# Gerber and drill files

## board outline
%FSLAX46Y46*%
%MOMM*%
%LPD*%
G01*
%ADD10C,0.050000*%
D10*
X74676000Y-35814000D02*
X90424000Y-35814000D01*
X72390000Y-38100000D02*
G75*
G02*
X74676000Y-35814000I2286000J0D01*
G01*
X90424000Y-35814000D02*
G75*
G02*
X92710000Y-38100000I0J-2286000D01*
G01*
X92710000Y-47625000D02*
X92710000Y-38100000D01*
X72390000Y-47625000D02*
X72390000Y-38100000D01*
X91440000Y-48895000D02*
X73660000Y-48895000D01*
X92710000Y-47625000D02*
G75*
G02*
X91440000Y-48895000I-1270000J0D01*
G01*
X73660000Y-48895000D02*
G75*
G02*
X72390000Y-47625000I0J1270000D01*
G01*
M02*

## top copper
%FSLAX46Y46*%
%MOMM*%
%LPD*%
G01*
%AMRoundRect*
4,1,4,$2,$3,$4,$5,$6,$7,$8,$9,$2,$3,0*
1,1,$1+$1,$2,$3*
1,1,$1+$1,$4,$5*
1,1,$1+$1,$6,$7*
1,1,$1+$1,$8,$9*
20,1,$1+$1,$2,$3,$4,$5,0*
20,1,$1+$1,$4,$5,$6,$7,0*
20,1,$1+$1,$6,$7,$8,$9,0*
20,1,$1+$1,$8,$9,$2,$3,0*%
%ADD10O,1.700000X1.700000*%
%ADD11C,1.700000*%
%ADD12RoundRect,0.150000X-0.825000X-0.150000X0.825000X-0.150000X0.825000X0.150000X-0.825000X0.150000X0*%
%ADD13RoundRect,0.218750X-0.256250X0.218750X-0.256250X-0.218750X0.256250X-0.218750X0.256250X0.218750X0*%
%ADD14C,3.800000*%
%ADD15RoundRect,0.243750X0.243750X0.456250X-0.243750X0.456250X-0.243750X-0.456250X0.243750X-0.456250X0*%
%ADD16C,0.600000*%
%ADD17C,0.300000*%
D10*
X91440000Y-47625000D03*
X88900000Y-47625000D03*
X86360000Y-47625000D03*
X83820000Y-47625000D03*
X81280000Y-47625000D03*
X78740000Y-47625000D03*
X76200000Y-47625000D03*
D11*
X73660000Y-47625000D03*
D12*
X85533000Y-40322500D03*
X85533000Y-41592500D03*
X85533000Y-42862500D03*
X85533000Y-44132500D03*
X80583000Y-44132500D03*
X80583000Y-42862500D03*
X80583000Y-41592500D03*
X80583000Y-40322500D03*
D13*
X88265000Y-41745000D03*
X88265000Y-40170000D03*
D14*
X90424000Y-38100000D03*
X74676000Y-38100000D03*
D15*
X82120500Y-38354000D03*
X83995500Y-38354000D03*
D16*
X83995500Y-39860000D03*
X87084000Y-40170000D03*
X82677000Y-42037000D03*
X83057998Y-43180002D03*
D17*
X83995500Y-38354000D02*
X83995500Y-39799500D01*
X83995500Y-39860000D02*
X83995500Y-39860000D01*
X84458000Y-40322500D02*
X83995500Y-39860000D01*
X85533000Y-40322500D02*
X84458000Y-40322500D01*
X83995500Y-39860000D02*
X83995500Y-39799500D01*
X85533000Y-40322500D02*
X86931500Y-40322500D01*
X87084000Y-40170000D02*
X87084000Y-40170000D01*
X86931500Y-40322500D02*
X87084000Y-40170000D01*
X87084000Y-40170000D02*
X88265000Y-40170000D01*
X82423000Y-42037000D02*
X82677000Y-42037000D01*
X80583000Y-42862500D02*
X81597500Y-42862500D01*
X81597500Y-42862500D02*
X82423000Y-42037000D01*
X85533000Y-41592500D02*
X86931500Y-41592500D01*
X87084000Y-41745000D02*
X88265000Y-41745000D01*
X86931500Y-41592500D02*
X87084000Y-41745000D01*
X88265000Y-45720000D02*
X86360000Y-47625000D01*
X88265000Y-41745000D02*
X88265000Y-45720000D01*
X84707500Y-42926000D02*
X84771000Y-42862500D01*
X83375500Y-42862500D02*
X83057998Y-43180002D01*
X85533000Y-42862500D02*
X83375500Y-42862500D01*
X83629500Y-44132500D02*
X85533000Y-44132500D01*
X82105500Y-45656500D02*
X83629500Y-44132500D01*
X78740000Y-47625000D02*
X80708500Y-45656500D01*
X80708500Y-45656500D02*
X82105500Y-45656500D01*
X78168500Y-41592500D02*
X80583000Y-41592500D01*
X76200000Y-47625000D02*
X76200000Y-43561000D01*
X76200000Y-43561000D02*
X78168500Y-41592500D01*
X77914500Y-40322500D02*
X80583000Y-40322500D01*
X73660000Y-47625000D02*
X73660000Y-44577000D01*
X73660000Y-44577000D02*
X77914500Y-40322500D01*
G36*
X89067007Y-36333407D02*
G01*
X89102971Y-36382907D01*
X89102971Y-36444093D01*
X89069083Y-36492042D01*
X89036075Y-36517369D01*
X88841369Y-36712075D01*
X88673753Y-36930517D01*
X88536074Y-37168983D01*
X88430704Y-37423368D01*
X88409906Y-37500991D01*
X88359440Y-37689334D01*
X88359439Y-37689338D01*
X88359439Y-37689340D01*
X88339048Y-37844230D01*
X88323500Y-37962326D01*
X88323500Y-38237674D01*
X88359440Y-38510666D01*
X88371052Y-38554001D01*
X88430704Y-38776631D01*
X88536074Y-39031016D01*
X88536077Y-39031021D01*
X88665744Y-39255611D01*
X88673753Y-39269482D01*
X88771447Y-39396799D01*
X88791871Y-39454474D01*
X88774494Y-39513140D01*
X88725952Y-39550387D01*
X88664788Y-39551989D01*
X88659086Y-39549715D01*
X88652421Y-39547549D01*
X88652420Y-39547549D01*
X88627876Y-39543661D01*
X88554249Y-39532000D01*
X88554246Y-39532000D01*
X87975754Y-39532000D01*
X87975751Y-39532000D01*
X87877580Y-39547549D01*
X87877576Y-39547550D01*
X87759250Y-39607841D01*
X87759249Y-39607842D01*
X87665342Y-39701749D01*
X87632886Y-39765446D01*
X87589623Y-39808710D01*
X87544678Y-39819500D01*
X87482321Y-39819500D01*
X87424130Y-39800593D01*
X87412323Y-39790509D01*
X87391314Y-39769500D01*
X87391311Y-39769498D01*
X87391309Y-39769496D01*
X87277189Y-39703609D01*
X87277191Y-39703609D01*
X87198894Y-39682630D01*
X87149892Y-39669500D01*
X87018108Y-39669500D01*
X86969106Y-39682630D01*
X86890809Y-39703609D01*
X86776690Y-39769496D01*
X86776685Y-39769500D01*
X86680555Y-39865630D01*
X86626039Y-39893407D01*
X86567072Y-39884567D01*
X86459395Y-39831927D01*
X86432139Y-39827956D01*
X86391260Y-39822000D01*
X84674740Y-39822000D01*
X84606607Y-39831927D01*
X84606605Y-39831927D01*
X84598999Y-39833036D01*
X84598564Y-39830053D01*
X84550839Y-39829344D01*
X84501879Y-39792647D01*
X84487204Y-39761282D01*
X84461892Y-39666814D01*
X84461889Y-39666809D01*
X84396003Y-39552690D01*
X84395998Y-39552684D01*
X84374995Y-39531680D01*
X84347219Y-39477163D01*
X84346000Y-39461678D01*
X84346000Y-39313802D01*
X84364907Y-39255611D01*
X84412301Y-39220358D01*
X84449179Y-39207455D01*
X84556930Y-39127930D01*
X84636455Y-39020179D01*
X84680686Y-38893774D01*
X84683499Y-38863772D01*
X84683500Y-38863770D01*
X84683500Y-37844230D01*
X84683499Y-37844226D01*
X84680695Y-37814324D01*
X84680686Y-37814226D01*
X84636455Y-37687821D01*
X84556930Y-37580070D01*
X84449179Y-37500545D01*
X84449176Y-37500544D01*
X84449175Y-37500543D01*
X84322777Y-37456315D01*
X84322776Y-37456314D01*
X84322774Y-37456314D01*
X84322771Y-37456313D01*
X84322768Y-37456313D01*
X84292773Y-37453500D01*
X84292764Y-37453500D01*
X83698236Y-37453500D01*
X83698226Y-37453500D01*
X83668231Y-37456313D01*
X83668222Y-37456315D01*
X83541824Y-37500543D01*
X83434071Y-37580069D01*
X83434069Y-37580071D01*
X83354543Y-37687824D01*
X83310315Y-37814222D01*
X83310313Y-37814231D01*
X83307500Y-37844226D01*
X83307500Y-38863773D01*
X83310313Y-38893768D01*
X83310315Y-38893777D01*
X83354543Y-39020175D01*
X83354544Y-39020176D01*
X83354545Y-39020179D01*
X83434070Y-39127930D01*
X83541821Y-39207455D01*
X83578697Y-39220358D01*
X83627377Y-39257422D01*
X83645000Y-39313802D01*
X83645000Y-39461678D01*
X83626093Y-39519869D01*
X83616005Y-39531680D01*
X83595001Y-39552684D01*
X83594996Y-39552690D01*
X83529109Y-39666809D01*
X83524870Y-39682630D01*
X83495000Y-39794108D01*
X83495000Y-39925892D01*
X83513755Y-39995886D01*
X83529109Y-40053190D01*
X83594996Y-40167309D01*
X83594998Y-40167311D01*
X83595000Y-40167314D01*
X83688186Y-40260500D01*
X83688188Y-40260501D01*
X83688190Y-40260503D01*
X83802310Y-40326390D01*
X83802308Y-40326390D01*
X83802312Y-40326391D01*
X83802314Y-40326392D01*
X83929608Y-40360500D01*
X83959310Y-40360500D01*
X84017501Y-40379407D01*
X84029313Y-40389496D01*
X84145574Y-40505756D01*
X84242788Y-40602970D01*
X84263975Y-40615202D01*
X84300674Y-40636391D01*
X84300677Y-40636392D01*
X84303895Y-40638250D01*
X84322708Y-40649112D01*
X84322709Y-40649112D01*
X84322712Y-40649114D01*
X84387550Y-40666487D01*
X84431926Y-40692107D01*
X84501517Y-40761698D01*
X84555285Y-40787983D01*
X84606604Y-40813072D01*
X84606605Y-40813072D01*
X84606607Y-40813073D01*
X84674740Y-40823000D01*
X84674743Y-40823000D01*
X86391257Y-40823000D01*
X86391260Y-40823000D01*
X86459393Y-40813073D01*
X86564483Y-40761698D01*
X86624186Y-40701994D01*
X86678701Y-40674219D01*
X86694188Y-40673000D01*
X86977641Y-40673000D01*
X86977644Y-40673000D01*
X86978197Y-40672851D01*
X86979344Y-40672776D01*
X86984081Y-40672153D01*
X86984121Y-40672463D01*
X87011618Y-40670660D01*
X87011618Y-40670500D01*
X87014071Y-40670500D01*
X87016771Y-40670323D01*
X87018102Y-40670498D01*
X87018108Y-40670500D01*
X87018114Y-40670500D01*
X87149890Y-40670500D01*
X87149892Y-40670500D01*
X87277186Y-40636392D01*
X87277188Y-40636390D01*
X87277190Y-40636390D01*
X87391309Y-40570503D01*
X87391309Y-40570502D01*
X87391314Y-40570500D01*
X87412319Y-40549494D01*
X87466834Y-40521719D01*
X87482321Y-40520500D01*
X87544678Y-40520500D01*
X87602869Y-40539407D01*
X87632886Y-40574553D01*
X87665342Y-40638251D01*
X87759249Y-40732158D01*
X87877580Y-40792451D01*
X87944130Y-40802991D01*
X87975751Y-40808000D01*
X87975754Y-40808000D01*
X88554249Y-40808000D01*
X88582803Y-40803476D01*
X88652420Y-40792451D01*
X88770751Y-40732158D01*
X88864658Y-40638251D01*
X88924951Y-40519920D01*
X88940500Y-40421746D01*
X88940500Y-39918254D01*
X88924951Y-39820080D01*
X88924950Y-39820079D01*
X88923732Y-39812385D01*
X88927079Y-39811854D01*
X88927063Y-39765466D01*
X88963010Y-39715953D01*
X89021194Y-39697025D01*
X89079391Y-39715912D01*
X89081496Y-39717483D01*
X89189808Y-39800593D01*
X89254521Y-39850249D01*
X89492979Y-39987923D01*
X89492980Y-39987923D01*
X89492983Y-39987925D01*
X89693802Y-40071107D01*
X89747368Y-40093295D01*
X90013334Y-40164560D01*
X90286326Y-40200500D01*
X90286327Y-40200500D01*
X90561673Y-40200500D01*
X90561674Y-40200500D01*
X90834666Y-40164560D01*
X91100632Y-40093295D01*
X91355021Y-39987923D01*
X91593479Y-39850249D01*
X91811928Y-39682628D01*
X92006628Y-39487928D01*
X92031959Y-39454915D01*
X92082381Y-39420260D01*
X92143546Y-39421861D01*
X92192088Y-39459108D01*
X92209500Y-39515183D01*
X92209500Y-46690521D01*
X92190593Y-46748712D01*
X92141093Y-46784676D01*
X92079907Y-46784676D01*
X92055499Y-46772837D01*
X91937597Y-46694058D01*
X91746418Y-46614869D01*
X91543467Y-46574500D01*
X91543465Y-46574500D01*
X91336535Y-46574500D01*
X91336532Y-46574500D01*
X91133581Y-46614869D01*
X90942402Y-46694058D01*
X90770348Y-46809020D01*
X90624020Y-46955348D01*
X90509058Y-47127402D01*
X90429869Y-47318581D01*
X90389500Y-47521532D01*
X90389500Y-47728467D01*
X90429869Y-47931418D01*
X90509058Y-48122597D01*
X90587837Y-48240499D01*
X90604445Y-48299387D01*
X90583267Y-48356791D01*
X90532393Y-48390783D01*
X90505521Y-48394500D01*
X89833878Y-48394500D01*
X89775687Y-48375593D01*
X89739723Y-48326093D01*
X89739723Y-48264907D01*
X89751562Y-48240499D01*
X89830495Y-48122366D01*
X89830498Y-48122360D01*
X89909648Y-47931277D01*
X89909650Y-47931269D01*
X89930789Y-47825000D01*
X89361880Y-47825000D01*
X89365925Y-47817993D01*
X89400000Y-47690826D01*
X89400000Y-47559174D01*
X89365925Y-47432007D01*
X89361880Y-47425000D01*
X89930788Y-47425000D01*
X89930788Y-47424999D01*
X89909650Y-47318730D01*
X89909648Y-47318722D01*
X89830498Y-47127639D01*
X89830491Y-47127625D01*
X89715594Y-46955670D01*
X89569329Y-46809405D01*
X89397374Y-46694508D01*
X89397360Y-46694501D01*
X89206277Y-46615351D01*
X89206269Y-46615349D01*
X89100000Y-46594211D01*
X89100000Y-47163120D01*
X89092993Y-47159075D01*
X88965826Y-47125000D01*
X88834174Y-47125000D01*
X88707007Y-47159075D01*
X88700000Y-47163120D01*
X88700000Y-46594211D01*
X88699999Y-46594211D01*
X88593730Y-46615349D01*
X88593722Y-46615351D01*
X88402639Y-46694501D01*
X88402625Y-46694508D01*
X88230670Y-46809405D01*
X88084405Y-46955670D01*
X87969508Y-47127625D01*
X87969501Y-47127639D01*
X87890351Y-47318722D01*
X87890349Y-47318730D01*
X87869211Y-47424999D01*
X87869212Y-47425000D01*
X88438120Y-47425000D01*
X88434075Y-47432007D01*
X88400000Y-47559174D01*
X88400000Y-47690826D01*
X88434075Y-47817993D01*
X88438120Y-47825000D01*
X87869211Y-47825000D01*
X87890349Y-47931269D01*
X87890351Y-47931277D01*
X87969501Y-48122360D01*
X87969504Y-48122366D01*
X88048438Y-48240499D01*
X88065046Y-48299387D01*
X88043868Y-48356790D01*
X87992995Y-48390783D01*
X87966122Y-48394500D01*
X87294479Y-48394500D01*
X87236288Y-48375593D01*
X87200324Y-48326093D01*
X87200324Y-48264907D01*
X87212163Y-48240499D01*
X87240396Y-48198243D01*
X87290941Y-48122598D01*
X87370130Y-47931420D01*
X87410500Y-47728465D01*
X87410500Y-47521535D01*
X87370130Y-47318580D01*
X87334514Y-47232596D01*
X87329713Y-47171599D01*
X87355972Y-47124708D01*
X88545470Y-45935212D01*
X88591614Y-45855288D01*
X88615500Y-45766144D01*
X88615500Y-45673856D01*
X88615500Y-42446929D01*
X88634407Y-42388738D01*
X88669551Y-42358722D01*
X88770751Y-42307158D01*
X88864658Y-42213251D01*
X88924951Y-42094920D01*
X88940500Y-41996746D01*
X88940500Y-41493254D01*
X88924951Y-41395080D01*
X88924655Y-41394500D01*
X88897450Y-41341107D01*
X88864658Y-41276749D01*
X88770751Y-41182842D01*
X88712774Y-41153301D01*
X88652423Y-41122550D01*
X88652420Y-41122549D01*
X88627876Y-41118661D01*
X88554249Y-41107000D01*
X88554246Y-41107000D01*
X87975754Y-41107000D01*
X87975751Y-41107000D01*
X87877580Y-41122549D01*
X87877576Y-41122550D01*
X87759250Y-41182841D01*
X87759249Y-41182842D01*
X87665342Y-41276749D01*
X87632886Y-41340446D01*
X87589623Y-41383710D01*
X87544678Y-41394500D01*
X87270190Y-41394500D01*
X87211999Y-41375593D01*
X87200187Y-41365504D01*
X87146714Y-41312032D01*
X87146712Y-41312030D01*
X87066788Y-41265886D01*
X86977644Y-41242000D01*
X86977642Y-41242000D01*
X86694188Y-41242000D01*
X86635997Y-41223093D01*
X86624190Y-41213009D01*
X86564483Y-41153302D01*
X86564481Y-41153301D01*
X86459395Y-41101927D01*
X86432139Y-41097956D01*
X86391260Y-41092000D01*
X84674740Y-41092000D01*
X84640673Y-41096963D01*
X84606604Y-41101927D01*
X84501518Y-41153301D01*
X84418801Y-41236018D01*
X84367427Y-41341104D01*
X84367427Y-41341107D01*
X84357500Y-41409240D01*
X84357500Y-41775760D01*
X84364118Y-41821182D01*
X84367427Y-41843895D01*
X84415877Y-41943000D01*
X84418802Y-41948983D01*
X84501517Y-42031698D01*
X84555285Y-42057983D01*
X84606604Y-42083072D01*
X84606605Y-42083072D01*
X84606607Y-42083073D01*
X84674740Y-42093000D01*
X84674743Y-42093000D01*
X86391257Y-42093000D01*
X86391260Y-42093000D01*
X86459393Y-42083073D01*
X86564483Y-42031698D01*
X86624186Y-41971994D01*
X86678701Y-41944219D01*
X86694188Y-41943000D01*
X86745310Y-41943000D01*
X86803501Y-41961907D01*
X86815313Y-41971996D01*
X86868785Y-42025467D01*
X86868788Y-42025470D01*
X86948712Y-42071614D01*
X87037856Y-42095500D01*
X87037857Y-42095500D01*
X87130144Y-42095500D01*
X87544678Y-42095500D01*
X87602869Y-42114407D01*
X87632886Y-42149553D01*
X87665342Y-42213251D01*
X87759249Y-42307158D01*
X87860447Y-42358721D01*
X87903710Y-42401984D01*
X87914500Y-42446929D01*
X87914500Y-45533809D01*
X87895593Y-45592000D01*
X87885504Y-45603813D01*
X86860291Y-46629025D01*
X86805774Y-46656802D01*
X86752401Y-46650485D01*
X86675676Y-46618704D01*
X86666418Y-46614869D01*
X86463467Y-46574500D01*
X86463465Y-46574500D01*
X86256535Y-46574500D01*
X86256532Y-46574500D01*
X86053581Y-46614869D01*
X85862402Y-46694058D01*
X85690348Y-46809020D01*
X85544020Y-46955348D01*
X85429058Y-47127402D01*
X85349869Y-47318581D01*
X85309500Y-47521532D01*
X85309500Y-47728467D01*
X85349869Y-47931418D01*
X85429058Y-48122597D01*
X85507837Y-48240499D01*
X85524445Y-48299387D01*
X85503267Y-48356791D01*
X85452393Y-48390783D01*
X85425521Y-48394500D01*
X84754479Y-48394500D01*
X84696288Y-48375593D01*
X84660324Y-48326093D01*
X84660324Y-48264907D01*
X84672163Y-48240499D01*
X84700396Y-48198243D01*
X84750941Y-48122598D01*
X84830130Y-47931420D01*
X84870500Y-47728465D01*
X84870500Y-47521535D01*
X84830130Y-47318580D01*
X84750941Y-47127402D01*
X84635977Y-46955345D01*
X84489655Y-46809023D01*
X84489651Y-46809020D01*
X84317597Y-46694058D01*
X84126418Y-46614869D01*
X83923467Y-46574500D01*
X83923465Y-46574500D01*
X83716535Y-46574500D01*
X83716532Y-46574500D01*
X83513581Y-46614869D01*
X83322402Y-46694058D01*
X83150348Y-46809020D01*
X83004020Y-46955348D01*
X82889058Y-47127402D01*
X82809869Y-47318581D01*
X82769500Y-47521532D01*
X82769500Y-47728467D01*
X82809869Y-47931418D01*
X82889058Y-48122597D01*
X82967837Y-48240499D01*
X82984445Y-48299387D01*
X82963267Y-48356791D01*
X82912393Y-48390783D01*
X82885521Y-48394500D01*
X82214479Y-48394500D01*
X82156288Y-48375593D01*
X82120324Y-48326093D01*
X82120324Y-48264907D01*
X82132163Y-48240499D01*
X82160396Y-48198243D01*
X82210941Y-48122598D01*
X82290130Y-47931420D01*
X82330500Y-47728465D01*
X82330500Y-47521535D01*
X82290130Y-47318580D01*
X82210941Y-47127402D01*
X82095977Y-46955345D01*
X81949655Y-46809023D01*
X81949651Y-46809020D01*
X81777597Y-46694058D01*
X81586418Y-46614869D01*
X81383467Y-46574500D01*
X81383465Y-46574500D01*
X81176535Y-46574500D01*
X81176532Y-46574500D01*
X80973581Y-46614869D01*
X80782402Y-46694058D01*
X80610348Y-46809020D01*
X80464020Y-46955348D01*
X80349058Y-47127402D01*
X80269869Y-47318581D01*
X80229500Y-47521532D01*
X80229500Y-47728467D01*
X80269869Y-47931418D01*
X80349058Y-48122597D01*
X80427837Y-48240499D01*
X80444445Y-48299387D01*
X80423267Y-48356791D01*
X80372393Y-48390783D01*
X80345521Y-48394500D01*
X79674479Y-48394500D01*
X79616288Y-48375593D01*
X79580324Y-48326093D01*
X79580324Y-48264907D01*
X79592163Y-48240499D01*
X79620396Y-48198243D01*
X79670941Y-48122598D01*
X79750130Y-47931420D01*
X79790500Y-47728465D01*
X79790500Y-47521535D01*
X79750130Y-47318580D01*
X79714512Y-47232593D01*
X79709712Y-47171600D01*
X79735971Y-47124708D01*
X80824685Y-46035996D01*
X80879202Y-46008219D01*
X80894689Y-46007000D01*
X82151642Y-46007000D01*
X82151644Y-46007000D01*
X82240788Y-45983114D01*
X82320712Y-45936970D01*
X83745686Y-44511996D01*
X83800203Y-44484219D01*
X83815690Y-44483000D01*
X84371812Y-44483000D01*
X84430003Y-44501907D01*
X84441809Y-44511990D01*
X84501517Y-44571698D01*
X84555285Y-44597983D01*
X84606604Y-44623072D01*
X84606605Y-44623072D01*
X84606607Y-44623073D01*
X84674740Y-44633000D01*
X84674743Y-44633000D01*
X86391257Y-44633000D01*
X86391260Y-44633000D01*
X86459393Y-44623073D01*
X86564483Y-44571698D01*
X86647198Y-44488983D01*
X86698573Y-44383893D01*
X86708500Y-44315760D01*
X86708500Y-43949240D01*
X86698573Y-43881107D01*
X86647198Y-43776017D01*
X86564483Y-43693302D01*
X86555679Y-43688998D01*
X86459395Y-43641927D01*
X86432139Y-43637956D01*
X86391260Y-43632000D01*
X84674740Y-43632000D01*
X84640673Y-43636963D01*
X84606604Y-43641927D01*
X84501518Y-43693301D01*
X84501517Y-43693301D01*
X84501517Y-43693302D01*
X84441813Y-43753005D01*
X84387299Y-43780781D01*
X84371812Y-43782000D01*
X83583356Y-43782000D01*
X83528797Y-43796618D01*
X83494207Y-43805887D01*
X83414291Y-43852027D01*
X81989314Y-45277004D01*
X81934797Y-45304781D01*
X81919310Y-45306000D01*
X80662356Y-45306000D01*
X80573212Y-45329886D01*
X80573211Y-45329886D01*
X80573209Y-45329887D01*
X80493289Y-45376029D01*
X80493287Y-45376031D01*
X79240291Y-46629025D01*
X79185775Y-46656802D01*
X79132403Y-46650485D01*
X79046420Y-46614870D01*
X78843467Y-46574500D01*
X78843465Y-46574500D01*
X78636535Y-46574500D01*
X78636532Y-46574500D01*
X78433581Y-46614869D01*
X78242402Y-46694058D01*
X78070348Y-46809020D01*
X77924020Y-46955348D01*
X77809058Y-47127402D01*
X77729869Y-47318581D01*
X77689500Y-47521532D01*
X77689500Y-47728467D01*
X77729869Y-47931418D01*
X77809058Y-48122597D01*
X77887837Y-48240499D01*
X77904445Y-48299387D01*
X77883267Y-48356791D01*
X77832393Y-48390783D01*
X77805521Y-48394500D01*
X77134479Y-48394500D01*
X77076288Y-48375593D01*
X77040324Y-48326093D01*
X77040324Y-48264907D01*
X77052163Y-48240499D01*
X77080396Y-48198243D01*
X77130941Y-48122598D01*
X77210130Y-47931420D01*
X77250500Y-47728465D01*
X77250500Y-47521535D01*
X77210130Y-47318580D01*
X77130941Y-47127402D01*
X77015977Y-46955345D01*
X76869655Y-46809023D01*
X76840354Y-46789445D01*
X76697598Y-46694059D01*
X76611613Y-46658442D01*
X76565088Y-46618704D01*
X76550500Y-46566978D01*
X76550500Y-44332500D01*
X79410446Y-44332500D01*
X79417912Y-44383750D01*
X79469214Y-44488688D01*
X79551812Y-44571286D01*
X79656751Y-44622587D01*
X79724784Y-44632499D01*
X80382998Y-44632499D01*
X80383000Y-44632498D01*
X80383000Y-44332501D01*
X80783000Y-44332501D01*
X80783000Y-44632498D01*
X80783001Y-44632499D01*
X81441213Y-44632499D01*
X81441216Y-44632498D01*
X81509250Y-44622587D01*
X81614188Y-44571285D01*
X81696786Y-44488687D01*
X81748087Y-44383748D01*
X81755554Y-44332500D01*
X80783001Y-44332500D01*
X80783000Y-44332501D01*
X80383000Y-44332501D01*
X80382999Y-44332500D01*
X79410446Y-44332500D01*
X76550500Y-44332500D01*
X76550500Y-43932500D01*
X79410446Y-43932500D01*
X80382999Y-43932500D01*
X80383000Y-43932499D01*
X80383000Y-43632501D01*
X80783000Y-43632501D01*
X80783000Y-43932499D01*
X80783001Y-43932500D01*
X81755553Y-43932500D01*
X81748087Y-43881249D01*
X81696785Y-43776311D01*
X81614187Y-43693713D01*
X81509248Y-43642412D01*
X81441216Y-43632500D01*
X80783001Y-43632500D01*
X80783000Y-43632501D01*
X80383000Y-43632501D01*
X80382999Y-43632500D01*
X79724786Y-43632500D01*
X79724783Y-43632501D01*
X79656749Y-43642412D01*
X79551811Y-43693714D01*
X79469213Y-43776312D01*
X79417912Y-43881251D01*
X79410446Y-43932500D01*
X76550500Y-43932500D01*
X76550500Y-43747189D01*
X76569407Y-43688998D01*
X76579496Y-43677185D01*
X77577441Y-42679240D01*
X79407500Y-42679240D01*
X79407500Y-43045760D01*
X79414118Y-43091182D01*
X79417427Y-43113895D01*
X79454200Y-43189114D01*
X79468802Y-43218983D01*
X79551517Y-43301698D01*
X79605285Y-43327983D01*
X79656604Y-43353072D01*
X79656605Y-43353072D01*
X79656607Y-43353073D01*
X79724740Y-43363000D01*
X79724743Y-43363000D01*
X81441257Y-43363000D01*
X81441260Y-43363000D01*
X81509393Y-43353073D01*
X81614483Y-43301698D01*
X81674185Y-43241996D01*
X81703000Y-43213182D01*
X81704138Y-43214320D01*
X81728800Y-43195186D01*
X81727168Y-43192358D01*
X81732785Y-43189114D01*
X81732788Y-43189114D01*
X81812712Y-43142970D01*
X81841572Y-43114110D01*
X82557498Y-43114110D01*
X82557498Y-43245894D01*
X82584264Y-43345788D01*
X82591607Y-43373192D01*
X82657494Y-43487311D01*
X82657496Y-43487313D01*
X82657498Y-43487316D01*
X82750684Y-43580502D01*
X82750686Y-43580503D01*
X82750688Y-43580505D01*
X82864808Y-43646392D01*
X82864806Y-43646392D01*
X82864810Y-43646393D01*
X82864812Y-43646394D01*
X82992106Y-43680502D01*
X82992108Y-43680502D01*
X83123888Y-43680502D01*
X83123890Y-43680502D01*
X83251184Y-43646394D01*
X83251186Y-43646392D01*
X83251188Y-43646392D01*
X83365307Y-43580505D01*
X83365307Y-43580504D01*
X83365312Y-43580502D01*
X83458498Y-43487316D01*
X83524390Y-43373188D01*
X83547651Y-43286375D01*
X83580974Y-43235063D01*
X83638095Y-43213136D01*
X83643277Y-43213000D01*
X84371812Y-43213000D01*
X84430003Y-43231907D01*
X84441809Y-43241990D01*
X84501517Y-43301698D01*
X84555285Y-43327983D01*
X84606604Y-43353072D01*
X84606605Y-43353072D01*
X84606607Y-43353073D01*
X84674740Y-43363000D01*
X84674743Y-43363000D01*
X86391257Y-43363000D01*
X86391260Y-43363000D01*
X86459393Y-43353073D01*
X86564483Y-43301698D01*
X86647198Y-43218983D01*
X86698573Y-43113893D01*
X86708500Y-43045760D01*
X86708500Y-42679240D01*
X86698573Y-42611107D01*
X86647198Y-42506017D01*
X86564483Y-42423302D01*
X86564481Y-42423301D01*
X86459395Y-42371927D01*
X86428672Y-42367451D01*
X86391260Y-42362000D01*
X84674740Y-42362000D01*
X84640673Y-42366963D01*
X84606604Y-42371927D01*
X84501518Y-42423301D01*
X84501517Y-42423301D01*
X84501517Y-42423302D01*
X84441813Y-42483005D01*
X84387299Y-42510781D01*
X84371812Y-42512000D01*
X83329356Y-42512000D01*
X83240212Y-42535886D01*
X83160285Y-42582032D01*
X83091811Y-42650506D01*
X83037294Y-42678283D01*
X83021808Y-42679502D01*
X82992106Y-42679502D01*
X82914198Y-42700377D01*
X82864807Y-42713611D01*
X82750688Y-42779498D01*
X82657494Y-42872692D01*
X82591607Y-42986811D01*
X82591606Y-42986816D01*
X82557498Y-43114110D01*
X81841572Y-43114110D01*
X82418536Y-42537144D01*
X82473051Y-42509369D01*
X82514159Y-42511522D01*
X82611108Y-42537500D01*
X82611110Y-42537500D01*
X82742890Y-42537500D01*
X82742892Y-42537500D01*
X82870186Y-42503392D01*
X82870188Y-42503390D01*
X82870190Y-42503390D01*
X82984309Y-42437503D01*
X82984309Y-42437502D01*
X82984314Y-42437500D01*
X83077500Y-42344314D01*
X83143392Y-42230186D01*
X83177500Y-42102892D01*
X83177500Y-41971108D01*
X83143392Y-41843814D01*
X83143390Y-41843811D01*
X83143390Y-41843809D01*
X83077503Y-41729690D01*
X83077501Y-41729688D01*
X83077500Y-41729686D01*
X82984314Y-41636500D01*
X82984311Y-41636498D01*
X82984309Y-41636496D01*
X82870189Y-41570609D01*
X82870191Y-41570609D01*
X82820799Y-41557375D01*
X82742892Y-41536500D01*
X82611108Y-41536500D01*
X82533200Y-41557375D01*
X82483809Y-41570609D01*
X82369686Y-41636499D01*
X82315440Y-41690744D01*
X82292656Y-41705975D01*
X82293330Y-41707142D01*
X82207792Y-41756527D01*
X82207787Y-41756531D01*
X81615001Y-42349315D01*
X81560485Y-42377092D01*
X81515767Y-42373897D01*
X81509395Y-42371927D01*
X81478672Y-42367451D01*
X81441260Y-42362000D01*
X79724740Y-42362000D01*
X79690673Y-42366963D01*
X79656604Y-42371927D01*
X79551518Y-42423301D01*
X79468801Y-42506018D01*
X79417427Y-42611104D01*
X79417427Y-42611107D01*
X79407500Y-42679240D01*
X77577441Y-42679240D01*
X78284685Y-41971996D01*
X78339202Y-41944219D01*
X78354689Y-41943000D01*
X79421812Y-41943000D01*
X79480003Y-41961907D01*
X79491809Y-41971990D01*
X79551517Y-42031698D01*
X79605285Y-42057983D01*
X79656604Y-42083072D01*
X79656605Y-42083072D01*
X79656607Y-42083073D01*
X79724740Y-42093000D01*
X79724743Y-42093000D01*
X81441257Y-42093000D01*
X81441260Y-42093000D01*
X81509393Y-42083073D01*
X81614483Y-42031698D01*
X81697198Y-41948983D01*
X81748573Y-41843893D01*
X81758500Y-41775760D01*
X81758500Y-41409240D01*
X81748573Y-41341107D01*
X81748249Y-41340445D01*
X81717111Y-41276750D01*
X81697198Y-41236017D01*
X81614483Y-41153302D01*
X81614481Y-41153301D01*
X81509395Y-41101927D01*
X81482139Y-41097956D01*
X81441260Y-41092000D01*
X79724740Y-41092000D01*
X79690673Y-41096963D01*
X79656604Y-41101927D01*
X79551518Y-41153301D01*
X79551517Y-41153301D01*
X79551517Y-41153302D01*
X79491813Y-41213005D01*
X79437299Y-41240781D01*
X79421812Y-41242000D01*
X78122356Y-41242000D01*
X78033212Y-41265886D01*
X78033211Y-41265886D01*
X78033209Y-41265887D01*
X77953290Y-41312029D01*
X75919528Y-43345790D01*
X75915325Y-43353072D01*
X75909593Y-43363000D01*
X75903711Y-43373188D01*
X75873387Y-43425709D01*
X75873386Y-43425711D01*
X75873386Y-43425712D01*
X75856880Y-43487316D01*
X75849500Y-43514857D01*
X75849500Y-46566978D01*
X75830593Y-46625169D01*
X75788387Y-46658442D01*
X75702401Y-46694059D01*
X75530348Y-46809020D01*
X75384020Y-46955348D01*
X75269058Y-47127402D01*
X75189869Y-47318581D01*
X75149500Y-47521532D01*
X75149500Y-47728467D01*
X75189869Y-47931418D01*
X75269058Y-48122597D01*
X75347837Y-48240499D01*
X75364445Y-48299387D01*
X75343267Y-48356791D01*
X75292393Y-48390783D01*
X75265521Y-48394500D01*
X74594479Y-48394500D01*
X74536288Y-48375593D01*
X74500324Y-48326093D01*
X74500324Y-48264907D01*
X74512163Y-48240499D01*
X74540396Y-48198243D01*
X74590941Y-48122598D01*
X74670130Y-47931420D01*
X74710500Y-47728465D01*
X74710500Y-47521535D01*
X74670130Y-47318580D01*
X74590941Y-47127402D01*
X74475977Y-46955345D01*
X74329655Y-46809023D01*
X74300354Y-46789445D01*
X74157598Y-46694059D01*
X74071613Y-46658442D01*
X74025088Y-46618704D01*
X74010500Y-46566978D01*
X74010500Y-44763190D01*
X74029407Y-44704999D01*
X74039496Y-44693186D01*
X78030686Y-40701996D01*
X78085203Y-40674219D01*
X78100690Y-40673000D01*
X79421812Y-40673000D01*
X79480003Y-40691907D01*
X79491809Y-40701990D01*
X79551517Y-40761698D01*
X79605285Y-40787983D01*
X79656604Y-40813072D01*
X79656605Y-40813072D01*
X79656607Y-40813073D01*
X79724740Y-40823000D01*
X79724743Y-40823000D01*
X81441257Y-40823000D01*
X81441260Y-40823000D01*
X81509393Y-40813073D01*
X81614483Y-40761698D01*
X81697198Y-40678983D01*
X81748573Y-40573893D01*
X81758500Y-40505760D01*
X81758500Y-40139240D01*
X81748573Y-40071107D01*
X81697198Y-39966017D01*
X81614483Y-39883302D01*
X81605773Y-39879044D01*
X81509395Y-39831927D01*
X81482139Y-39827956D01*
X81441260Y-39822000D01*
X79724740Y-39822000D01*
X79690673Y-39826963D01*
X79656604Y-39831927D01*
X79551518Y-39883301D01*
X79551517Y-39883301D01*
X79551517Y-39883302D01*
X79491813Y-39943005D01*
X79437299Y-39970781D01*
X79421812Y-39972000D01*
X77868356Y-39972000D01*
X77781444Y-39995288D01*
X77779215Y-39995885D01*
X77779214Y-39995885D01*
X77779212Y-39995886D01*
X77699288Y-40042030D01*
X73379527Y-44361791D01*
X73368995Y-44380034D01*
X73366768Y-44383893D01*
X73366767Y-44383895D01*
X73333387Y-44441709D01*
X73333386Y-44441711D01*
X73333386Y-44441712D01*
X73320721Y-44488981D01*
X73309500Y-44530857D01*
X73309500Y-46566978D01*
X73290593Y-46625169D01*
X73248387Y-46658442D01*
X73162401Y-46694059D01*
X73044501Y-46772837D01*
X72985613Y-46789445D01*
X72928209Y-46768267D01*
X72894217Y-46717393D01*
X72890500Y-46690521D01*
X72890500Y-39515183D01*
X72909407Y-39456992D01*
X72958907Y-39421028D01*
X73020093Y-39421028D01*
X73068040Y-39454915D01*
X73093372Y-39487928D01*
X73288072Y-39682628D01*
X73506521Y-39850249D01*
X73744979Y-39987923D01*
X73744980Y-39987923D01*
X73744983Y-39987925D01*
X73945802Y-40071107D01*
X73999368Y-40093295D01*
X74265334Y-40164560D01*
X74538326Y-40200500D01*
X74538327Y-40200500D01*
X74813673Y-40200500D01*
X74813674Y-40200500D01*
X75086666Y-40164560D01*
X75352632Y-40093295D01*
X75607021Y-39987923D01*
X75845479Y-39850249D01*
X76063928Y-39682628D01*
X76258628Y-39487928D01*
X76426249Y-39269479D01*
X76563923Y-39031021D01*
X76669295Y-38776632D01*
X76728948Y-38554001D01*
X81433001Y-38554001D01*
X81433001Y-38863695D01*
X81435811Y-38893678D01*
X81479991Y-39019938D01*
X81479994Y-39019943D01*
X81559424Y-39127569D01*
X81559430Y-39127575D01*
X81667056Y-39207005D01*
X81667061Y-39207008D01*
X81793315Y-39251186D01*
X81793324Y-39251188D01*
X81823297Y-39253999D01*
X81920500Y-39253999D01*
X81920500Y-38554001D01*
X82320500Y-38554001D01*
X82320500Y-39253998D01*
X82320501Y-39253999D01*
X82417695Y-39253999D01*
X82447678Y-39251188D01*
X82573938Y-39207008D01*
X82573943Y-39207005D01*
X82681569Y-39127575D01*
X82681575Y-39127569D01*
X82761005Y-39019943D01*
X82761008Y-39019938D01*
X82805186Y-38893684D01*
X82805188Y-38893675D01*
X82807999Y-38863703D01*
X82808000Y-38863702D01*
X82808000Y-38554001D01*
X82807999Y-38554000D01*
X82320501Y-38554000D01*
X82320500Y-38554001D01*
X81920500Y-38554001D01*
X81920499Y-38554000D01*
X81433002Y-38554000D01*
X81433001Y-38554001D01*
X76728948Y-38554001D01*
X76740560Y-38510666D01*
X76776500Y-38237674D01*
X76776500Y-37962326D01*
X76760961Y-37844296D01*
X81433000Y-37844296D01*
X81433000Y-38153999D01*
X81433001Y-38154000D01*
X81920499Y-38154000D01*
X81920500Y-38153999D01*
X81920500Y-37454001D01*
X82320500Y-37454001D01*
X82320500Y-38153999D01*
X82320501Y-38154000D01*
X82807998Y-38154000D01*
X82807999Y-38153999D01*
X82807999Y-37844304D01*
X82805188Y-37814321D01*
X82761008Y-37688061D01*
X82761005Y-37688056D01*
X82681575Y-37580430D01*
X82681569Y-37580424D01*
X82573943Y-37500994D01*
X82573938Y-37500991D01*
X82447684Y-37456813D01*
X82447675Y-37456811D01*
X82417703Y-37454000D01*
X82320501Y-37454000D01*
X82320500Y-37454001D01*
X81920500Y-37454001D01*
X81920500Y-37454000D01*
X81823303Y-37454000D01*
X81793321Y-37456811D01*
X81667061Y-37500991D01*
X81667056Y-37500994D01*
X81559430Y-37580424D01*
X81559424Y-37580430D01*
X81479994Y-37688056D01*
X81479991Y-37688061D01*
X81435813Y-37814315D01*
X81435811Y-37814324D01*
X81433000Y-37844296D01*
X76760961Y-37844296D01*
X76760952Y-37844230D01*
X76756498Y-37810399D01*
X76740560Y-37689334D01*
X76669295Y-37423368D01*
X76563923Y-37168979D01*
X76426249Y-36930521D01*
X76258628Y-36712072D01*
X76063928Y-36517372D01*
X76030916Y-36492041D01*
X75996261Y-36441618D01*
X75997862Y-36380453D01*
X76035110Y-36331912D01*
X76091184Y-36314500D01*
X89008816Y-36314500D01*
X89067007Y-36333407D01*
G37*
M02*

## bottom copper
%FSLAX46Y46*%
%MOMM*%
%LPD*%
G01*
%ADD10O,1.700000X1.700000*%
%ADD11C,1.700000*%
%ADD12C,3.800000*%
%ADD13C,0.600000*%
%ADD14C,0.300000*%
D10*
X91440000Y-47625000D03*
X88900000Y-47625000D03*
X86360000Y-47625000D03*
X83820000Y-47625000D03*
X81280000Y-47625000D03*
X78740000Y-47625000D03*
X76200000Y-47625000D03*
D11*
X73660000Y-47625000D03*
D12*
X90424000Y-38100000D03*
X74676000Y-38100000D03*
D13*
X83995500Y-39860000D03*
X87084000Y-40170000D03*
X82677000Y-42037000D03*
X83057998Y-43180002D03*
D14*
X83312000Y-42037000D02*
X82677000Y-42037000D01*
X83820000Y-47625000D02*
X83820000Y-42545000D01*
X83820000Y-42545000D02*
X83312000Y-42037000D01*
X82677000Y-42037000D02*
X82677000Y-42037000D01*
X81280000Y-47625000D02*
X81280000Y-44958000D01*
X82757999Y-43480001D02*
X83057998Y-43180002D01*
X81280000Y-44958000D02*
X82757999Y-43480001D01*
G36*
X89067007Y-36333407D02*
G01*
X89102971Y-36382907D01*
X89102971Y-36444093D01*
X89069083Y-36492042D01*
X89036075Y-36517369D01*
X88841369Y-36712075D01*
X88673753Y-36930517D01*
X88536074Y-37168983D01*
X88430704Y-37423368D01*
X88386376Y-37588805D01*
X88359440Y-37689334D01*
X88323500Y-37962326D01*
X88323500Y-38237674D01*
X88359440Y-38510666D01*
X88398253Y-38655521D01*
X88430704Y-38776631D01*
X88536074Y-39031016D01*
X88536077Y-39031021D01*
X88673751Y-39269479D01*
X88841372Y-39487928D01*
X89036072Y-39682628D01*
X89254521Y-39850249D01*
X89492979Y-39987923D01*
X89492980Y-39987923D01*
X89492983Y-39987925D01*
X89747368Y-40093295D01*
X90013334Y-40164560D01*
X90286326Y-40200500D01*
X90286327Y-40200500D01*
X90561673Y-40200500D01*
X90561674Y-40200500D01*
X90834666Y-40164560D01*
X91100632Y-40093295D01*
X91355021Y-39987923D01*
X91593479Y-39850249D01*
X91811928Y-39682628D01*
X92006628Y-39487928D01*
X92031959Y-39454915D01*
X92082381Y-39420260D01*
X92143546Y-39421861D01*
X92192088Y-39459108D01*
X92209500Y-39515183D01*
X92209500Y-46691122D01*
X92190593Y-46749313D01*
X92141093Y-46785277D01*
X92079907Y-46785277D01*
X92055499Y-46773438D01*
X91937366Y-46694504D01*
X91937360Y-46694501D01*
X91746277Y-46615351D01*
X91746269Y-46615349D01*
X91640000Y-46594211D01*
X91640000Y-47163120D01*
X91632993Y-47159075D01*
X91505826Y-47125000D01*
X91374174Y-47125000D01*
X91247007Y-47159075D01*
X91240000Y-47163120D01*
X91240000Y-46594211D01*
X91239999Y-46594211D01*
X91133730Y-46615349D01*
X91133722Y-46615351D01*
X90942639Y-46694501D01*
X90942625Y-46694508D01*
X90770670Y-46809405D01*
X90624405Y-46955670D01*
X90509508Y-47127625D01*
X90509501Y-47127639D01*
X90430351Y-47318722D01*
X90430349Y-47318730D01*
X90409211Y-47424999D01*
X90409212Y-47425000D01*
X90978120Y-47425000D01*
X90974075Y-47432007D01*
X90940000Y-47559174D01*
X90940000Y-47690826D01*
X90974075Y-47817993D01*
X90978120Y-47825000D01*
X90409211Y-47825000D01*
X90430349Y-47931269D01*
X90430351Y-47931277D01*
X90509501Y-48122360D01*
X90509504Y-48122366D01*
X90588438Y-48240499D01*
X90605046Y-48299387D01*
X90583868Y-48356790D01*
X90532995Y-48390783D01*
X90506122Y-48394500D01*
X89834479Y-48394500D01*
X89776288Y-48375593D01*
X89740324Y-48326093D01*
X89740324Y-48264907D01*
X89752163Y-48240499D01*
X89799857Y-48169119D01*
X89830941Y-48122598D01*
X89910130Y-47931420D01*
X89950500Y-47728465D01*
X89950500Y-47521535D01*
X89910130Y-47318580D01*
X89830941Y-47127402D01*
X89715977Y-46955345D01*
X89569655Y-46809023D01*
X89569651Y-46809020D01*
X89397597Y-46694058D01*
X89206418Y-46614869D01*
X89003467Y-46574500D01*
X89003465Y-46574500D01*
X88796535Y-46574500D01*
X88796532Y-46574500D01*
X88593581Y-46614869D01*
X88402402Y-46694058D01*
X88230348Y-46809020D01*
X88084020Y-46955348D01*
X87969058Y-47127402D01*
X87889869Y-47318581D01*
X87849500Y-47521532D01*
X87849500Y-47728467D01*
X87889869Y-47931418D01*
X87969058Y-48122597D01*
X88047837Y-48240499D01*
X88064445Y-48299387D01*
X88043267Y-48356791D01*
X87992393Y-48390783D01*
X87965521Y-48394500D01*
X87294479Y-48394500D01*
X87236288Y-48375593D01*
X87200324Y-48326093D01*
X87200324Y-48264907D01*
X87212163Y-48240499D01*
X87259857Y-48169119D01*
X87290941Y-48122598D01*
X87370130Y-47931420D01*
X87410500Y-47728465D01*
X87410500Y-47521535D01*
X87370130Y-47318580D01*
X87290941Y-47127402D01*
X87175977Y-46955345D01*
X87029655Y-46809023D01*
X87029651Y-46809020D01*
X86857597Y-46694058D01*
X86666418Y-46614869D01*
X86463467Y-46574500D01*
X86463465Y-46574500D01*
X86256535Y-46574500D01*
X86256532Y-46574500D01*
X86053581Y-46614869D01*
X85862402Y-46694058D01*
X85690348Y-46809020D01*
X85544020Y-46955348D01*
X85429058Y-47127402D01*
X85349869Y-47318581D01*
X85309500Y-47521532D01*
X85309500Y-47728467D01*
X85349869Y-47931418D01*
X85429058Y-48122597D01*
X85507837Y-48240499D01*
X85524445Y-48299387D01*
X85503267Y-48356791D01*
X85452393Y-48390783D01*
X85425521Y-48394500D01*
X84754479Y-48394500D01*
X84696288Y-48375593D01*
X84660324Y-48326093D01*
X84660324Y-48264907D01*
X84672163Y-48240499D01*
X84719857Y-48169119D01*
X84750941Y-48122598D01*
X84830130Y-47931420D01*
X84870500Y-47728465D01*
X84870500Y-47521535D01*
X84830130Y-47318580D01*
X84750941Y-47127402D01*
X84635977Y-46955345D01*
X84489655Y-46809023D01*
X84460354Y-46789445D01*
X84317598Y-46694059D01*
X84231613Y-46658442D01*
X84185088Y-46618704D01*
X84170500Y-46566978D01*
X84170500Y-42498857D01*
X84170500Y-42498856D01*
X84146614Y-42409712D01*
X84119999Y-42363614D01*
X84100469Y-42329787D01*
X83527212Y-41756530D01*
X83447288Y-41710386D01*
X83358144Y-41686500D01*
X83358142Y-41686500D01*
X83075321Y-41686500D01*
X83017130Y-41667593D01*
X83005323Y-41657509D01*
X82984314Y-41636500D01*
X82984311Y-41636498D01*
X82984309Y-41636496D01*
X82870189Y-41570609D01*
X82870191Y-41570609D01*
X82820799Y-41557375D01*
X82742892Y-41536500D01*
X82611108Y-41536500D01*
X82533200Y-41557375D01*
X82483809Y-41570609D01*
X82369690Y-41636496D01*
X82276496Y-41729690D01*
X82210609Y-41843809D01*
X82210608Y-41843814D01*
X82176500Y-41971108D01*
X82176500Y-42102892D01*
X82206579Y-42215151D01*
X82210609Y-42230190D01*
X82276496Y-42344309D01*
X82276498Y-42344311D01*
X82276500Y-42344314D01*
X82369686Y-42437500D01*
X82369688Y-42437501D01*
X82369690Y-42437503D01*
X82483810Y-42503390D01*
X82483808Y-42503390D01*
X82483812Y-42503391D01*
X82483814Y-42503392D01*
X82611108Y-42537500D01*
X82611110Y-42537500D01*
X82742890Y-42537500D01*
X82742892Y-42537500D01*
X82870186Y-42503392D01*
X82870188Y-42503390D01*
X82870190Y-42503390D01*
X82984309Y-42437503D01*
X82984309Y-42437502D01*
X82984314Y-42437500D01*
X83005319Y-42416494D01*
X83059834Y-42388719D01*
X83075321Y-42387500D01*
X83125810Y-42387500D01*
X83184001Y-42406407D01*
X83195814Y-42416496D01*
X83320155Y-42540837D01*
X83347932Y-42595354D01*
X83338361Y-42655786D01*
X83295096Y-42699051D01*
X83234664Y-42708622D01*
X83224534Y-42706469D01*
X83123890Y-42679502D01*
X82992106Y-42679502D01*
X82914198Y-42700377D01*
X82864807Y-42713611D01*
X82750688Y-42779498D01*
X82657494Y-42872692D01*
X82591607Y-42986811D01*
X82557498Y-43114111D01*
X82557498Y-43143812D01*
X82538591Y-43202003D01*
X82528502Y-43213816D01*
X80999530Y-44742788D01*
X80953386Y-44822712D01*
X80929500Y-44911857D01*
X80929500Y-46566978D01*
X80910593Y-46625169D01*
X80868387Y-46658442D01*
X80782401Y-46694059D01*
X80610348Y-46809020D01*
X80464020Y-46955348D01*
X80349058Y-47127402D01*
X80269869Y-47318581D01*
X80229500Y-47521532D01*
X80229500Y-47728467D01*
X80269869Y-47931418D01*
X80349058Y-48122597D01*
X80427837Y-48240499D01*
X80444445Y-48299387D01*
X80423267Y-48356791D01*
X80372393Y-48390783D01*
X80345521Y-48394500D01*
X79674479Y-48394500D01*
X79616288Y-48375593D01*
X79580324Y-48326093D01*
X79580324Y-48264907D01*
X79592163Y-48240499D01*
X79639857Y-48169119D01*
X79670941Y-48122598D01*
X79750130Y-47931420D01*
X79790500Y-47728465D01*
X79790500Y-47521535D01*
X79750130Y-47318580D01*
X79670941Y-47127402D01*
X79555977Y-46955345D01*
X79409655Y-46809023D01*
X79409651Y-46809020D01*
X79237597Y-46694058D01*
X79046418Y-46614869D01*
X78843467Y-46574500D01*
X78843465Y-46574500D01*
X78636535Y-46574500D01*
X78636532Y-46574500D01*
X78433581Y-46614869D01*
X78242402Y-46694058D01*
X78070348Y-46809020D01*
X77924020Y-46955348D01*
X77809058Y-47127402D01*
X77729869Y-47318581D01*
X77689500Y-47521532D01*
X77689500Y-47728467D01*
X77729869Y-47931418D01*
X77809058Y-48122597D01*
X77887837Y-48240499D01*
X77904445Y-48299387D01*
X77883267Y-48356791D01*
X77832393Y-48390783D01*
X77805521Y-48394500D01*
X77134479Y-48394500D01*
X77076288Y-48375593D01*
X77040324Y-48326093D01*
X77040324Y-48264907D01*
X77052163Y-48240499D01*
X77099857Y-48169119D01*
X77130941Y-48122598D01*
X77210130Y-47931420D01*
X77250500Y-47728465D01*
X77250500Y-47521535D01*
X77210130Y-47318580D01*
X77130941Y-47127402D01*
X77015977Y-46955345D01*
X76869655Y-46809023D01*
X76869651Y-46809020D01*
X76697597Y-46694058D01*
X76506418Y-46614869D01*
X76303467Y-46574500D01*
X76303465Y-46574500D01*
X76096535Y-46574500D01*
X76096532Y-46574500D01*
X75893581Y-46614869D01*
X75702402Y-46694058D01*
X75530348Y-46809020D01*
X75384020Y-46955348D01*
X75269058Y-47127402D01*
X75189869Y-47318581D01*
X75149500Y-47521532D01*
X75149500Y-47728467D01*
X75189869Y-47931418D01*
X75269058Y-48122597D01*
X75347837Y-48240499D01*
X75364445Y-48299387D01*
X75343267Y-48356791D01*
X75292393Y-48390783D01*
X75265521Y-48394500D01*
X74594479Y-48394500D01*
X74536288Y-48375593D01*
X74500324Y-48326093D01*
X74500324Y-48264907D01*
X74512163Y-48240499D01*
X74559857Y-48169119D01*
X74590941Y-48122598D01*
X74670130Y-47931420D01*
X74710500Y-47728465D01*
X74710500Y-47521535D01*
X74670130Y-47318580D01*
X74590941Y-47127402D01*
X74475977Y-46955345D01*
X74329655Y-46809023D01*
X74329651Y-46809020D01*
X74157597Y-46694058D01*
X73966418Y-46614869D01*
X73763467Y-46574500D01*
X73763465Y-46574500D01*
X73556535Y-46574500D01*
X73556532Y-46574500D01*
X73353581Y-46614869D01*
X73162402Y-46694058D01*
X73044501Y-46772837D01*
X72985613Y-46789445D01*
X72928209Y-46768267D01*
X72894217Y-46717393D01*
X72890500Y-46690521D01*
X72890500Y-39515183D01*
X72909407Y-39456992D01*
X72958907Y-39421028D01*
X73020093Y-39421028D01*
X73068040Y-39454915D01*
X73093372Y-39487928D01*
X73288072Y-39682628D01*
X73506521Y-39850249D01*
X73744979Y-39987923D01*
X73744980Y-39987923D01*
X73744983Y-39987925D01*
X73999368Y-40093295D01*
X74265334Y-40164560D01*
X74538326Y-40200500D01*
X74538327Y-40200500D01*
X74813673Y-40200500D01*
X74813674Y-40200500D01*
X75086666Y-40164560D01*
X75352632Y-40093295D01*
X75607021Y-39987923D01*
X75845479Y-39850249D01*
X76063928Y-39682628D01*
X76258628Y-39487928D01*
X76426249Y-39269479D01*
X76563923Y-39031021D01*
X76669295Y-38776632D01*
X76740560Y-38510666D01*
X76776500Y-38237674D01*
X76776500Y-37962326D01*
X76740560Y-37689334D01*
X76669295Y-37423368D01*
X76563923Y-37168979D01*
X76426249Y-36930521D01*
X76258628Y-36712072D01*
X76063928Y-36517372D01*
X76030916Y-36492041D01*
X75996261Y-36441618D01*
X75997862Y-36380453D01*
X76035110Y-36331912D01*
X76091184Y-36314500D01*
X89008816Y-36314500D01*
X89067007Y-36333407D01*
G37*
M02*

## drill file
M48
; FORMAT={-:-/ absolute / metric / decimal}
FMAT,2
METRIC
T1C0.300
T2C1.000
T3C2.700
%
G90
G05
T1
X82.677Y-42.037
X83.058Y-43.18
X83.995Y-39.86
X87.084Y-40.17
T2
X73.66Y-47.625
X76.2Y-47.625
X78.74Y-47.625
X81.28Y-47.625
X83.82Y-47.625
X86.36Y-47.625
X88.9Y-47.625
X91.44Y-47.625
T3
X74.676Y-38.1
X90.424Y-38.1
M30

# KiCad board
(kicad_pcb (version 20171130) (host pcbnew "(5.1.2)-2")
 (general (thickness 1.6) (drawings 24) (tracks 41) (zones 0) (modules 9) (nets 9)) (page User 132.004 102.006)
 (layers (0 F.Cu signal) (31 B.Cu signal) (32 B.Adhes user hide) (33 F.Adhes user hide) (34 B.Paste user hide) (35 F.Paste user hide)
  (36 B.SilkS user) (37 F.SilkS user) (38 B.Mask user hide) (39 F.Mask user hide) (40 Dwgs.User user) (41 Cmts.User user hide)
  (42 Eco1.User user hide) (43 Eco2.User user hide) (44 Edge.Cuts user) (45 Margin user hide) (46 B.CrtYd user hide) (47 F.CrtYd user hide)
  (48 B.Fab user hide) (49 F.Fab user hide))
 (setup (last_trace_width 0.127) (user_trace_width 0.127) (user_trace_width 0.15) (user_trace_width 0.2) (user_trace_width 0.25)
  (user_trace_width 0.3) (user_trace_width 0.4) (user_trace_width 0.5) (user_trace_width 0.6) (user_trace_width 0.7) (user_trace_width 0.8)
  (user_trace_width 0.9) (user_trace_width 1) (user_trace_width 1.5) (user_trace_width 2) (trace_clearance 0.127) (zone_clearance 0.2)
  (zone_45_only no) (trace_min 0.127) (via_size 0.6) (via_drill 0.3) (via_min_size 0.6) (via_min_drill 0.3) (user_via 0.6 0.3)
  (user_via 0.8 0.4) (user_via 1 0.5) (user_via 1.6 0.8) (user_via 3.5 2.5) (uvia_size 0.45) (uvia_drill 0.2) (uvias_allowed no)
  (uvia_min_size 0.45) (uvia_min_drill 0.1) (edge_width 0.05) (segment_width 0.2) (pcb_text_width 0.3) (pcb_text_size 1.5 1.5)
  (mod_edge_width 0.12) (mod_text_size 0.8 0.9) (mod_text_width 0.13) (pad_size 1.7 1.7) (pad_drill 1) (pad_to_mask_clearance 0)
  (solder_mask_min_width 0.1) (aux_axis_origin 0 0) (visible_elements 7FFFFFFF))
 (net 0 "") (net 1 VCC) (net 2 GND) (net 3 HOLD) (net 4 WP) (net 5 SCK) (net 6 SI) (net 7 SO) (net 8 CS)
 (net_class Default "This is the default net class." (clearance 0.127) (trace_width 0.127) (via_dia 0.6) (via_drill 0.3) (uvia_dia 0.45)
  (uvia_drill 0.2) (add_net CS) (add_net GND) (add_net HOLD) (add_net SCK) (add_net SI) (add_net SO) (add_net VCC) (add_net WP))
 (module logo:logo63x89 (layer B.Cu) (at 82.55 39.116 180)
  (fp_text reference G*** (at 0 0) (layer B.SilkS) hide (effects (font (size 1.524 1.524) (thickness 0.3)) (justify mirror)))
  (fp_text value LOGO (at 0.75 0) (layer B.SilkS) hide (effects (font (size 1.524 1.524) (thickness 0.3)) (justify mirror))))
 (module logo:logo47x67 (layer F.Cu) (at 90.551 42.799)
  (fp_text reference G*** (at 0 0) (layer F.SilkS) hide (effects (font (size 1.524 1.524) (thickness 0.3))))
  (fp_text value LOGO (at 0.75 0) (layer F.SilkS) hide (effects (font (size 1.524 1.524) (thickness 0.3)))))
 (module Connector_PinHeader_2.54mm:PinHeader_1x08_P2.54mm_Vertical (layer B.Cu) (at 73.66 47.625 270)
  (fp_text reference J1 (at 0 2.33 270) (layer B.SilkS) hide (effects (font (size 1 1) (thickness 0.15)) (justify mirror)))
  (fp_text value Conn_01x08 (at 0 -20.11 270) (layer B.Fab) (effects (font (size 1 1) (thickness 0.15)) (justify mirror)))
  (pad 8 thru_hole oval (at 0 -17.78 270) (size 1.7 1.7) (drill 1) (layers *.Cu *.Mask) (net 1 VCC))
  (pad 7 thru_hole oval (at 0 -15.24 270) (size 1.7 1.7) (drill 1) (layers *.Cu *.Mask) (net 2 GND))
  (pad 6 thru_hole oval (at 0 -12.7 270) (size 1.7 1.7) (drill 1) (layers *.Cu *.Mask) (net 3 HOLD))
  (pad 5 thru_hole oval (at 0 -10.16 270) (size 1.7 1.7) (drill 1) (layers *.Cu *.Mask) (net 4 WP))
  (pad 4 thru_hole oval (at 0 -7.62 270) (size 1.7 1.7) (drill 1) (layers *.Cu *.Mask) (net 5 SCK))
  (pad 3 thru_hole oval (at 0 -5.08 270) (size 1.7 1.7) (drill 1) (layers *.Cu *.Mask) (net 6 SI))
  (pad 2 thru_hole oval (at 0 -2.54 270) (size 1.7 1.7) (drill 1) (layers *.Cu *.Mask) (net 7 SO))
  (pad 1 thru_hole circle (at 0 0 270) (size 1.7 1.7) (drill 1) (layers *.Cu *.Mask) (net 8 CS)))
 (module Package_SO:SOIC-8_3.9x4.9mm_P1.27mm (layer F.Cu) (at 83.058 42.2275)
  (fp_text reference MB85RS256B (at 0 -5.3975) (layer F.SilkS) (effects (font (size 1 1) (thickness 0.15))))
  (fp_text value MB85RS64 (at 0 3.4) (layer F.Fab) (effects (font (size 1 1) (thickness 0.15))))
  (pad 8 smd roundrect (at 2.475 -1.905) (size 1.95 0.6) (layers F.Cu F.Paste F.Mask) (roundrect_rratio 0.25) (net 1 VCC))
  (pad 7 smd roundrect (at 2.475 -0.635) (size 1.95 0.6) (layers F.Cu F.Paste F.Mask) (roundrect_rratio 0.25) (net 3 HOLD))
  (pad 6 smd roundrect (at 2.475 0.635) (size 1.95 0.6) (layers F.Cu F.Paste F.Mask) (roundrect_rratio 0.25) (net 5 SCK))
  (pad 5 smd roundrect (at 2.475 1.905) (size 1.95 0.6) (layers F.Cu F.Paste F.Mask) (roundrect_rratio 0.25) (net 6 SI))
  (pad 4 smd roundrect (at -2.475 1.905) (size 1.95 0.6) (layers F.Cu F.Paste F.Mask) (roundrect_rratio 0.25) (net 2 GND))
  (pad 3 smd roundrect (at -2.475 0.635) (size 1.95 0.6) (layers F.Cu F.Paste F.Mask) (roundrect_rratio 0.25) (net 4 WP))
  (pad 2 smd roundrect (at -2.475 -0.635) (size 1.95 0.6) (layers F.Cu F.Paste F.Mask) (roundrect_rratio 0.25) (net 7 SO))
  (pad 1 smd roundrect (at -2.475 -1.905) (size 1.95 0.6) (layers F.Cu F.Paste F.Mask) (roundrect_rratio 0.25) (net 8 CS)))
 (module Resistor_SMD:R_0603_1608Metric (layer F.Cu) (at 88.265 40.9575 270)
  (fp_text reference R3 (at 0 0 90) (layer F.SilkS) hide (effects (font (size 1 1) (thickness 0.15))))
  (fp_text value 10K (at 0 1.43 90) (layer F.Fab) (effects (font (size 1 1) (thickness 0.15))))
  (pad 2 smd roundrect (at 0.7875 0 270) (size 0.875 0.95) (layers F.Cu F.Paste F.Mask) (roundrect_rratio 0.25) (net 3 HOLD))
  (pad 1 smd roundrect (at -0.7875 0 270) (size 0.875 0.95) (layers F.Cu F.Paste F.Mask) (roundrect_rratio 0.25) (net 1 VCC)))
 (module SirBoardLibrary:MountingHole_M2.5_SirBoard (layer F.Cu) (at 90.424 38.1)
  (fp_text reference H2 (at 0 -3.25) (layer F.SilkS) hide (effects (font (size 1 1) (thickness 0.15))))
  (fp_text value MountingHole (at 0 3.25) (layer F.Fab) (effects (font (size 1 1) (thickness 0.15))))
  (pad 1 thru_hole circle (at 0 0) (size 3.8 3.8) (drill 2.7) (layers *.Cu *.Mask)))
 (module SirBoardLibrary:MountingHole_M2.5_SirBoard (layer F.Cu) (at 74.676 38.1)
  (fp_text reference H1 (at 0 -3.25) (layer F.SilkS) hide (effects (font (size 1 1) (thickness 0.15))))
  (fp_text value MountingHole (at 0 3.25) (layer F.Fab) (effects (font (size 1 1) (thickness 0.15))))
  (pad 1 thru_hole circle (at 0 0) (size 3.8 3.8) (drill 2.7) (layers *.Cu *.Mask)))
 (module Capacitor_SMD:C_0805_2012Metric (layer F.Cu) (at 83.058 38.354 180)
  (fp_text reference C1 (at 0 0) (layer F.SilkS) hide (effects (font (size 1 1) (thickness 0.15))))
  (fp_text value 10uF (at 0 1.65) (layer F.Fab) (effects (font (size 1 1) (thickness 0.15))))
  (pad 2 smd roundrect (at 0.9375 0 180) (size 0.975 1.4) (layers F.Cu F.Paste F.Mask) (roundrect_rratio 0.25) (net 2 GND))
  (pad 1 smd roundrect (at -0.9375 0 180) (size 0.975 1.4) (layers F.Cu F.Paste F.Mask) (roundrect_rratio 0.25) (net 1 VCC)))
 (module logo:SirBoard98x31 (layer B.Cu) (at 82.55 44.323 180)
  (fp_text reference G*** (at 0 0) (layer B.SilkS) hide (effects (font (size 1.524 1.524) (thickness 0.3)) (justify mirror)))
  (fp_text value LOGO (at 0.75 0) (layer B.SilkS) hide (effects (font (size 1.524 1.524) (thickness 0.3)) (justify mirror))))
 (gr_line (start 74.676 35.814) (end 90.424 35.814) (layer Edge.Cuts) (width 0.05))
 (gr_arc (start 74.676 38.1) (end 74.676 35.814) (angle -90) (layer Edge.Cuts) (width 0.05))
 (gr_arc (start 90.424 38.1) (end 92.71 38.1) (angle -90) (layer Edge.Cuts) (width 0.05))
 (gr_line (start 92.71 47.625) (end 92.71 38.1) (layer Edge.Cuts) (width 0.05))
 (gr_line (start 72.39 47.625) (end 72.39 38.1) (layer Edge.Cuts) (width 0.05))
 (gr_line (start 91.44 48.895) (end 73.66 48.895) (layer Edge.Cuts) (width 0.05))
 (gr_arc (start 91.44 47.625) (end 91.44 48.895) (angle -90) (layer Edge.Cuts) (width 0.05))
 (gr_arc (start 73.66 47.625) (end 72.39 47.625) (angle -90) (layer Edge.Cuts) (width 0.05))
 (segment (start 83.9955 38.354) (end 83.9955 39.7995) (width 0.3) (layer F.Cu) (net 1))
 (segment (start 83.9955 39.86) (end 83.9955 39.86) (width 0.3) (layer F.Cu) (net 1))
 (segment (start 84.458 40.3225) (end 83.9955 39.86) (width 0.3) (layer F.Cu) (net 1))
 (segment (start 85.533 40.3225) (end 84.458 40.3225) (width 0.3) (layer F.Cu) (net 1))
 (segment (start 83.9955 39.86) (end 83.9955 39.7995) (width 0.3) (layer F.Cu) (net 1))
 (via (at 83.9955 39.86) (size 0.6) (drill 0.3) (layers F.Cu B.Cu) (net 1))
 (segment (start 85.533 40.3225) (end 86.9315 40.3225) (width 0.3) (layer F.Cu) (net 1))
 (segment (start 87.084 40.17) (end 87.084 40.17) (width 0.3) (layer F.Cu) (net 1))
 (segment (start 86.9315 40.3225) (end 87.084 40.17) (width 0.3) (layer F.Cu) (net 1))
 (segment (start 87.084 40.17) (end 88.265 40.17) (width 0.3) (layer F.Cu) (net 1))
 (via (at 87.084 40.17) (size 0.6) (drill 0.3) (layers F.Cu B.Cu) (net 1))
 (segment (start 83.312 42.037) (end 82.677 42.037) (width 0.3) (layer B.Cu) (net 4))
 (segment (start 83.82 47.625) (end 83.82 42.545) (width 0.3) (layer B.Cu) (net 4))
 (segment (start 83.82 42.545) (end 83.312 42.037) (width 0.3) (layer B.Cu) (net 4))
 (segment (start 82.677 42.037) (end 82.677 42.037) (width 0.3) (layer B.Cu) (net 4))
 (via (at 82.677 42.037) (size 0.6) (drill 0.3) (layers F.Cu B.Cu) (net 4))
 (segment (start 82.423 42.037) (end 82.677 42.037) (width 0.3) (layer F.Cu) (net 4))
 (segment (start 80.583 42.8625) (end 81.5975 42.8625) (width 0.3) (layer F.Cu) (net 4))
 (segment (start 81.5975 42.8625) (end 82.423 42.037) (width 0.3) (layer F.Cu) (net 4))
 (segment (start 85.533 41.5925) (end 86.9315 41.5925) (width 0.3) (layer F.Cu) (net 3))
 (segment (start 87.084 41.745) (end 88.265 41.745) (width 0.3) (layer F.Cu) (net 3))
 (segment (start 86.9315 41.5925) (end 87.084 41.745) (width 0.3) (layer F.Cu) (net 3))
 (segment (start 88.265 45.72) (end 86.36 47.625) (width 0.3) (layer F.Cu) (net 3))
 (segment (start 88.265 41.745) (end 88.265 45.72) (width 0.3) (layer F.Cu) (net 3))
 (segment (start 84.7075 42.926) (end 84.771 42.8625) (width 0.3) (layer F.Cu) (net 5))
 (via (at 83.057998 43.180002) (size 0.6) (drill 0.3) (layers F.Cu B.Cu) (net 5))
 (segment (start 81.28 47.625) (end 81.28 44.958) (width 0.3) (layer B.Cu) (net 5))
 (segment (start 82.757999 43.480001) (end 83.057998 43.180002) (width 0.3) (layer B.Cu) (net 5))
 (segment (start 81.28 44.958) (end 82.757999 43.480001) (width 0.3) (layer B.Cu) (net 5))
 (segment (start 83.3755 42.8625) (end 83.057998 43.180002) (width 0.3) (layer F.Cu) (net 5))
 (segment (start 85.533 42.8625) (end 83.3755 42.8625) (width 0.3) (layer F.Cu) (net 5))
 (segment (start 83.6295 44.1325) (end 85.533 44.1325) (width 0.3) (layer F.Cu) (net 6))
 (segment (start 82.1055 45.6565) (end 83.6295 44.1325) (width 0.3) (layer F.Cu) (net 6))
 (segment (start 78.74 47.625) (end 80.7085 45.6565) (width 0.3) (layer F.Cu) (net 6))
 (segment (start 80.7085 45.6565) (end 82.1055 45.6565) (width 0.3) (layer F.Cu) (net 6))
 (segment (start 78.1685 41.5925) (end 80.583 41.5925) (width 0.3) (layer F.Cu) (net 7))
 (segment (start 76.2 47.625) (end 76.2 43.561) (width 0.3) (layer F.Cu) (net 7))
 (segment (start 76.2 43.561) (end 78.1685 41.5925) (width 0.3) (layer F.Cu) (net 7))
 (segment (start 77.9145 40.3225) (end 80.583 40.3225) (width 0.3) (layer F.Cu) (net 8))
 (segment (start 73.66 47.625) (end 73.66 44.577) (width 0.3) (layer F.Cu) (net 8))
 (segment (start 73.66 44.577) (end 77.9145 40.3225) (width 0.3) (layer F.Cu) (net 8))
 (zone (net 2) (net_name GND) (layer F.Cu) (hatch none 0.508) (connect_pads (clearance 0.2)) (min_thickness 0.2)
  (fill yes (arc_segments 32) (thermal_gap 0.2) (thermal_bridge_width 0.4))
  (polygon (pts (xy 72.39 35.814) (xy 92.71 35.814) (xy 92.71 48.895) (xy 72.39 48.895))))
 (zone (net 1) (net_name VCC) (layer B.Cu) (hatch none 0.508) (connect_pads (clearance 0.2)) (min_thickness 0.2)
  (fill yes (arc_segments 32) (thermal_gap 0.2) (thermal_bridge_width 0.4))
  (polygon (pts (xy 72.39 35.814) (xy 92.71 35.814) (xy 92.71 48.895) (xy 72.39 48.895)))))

